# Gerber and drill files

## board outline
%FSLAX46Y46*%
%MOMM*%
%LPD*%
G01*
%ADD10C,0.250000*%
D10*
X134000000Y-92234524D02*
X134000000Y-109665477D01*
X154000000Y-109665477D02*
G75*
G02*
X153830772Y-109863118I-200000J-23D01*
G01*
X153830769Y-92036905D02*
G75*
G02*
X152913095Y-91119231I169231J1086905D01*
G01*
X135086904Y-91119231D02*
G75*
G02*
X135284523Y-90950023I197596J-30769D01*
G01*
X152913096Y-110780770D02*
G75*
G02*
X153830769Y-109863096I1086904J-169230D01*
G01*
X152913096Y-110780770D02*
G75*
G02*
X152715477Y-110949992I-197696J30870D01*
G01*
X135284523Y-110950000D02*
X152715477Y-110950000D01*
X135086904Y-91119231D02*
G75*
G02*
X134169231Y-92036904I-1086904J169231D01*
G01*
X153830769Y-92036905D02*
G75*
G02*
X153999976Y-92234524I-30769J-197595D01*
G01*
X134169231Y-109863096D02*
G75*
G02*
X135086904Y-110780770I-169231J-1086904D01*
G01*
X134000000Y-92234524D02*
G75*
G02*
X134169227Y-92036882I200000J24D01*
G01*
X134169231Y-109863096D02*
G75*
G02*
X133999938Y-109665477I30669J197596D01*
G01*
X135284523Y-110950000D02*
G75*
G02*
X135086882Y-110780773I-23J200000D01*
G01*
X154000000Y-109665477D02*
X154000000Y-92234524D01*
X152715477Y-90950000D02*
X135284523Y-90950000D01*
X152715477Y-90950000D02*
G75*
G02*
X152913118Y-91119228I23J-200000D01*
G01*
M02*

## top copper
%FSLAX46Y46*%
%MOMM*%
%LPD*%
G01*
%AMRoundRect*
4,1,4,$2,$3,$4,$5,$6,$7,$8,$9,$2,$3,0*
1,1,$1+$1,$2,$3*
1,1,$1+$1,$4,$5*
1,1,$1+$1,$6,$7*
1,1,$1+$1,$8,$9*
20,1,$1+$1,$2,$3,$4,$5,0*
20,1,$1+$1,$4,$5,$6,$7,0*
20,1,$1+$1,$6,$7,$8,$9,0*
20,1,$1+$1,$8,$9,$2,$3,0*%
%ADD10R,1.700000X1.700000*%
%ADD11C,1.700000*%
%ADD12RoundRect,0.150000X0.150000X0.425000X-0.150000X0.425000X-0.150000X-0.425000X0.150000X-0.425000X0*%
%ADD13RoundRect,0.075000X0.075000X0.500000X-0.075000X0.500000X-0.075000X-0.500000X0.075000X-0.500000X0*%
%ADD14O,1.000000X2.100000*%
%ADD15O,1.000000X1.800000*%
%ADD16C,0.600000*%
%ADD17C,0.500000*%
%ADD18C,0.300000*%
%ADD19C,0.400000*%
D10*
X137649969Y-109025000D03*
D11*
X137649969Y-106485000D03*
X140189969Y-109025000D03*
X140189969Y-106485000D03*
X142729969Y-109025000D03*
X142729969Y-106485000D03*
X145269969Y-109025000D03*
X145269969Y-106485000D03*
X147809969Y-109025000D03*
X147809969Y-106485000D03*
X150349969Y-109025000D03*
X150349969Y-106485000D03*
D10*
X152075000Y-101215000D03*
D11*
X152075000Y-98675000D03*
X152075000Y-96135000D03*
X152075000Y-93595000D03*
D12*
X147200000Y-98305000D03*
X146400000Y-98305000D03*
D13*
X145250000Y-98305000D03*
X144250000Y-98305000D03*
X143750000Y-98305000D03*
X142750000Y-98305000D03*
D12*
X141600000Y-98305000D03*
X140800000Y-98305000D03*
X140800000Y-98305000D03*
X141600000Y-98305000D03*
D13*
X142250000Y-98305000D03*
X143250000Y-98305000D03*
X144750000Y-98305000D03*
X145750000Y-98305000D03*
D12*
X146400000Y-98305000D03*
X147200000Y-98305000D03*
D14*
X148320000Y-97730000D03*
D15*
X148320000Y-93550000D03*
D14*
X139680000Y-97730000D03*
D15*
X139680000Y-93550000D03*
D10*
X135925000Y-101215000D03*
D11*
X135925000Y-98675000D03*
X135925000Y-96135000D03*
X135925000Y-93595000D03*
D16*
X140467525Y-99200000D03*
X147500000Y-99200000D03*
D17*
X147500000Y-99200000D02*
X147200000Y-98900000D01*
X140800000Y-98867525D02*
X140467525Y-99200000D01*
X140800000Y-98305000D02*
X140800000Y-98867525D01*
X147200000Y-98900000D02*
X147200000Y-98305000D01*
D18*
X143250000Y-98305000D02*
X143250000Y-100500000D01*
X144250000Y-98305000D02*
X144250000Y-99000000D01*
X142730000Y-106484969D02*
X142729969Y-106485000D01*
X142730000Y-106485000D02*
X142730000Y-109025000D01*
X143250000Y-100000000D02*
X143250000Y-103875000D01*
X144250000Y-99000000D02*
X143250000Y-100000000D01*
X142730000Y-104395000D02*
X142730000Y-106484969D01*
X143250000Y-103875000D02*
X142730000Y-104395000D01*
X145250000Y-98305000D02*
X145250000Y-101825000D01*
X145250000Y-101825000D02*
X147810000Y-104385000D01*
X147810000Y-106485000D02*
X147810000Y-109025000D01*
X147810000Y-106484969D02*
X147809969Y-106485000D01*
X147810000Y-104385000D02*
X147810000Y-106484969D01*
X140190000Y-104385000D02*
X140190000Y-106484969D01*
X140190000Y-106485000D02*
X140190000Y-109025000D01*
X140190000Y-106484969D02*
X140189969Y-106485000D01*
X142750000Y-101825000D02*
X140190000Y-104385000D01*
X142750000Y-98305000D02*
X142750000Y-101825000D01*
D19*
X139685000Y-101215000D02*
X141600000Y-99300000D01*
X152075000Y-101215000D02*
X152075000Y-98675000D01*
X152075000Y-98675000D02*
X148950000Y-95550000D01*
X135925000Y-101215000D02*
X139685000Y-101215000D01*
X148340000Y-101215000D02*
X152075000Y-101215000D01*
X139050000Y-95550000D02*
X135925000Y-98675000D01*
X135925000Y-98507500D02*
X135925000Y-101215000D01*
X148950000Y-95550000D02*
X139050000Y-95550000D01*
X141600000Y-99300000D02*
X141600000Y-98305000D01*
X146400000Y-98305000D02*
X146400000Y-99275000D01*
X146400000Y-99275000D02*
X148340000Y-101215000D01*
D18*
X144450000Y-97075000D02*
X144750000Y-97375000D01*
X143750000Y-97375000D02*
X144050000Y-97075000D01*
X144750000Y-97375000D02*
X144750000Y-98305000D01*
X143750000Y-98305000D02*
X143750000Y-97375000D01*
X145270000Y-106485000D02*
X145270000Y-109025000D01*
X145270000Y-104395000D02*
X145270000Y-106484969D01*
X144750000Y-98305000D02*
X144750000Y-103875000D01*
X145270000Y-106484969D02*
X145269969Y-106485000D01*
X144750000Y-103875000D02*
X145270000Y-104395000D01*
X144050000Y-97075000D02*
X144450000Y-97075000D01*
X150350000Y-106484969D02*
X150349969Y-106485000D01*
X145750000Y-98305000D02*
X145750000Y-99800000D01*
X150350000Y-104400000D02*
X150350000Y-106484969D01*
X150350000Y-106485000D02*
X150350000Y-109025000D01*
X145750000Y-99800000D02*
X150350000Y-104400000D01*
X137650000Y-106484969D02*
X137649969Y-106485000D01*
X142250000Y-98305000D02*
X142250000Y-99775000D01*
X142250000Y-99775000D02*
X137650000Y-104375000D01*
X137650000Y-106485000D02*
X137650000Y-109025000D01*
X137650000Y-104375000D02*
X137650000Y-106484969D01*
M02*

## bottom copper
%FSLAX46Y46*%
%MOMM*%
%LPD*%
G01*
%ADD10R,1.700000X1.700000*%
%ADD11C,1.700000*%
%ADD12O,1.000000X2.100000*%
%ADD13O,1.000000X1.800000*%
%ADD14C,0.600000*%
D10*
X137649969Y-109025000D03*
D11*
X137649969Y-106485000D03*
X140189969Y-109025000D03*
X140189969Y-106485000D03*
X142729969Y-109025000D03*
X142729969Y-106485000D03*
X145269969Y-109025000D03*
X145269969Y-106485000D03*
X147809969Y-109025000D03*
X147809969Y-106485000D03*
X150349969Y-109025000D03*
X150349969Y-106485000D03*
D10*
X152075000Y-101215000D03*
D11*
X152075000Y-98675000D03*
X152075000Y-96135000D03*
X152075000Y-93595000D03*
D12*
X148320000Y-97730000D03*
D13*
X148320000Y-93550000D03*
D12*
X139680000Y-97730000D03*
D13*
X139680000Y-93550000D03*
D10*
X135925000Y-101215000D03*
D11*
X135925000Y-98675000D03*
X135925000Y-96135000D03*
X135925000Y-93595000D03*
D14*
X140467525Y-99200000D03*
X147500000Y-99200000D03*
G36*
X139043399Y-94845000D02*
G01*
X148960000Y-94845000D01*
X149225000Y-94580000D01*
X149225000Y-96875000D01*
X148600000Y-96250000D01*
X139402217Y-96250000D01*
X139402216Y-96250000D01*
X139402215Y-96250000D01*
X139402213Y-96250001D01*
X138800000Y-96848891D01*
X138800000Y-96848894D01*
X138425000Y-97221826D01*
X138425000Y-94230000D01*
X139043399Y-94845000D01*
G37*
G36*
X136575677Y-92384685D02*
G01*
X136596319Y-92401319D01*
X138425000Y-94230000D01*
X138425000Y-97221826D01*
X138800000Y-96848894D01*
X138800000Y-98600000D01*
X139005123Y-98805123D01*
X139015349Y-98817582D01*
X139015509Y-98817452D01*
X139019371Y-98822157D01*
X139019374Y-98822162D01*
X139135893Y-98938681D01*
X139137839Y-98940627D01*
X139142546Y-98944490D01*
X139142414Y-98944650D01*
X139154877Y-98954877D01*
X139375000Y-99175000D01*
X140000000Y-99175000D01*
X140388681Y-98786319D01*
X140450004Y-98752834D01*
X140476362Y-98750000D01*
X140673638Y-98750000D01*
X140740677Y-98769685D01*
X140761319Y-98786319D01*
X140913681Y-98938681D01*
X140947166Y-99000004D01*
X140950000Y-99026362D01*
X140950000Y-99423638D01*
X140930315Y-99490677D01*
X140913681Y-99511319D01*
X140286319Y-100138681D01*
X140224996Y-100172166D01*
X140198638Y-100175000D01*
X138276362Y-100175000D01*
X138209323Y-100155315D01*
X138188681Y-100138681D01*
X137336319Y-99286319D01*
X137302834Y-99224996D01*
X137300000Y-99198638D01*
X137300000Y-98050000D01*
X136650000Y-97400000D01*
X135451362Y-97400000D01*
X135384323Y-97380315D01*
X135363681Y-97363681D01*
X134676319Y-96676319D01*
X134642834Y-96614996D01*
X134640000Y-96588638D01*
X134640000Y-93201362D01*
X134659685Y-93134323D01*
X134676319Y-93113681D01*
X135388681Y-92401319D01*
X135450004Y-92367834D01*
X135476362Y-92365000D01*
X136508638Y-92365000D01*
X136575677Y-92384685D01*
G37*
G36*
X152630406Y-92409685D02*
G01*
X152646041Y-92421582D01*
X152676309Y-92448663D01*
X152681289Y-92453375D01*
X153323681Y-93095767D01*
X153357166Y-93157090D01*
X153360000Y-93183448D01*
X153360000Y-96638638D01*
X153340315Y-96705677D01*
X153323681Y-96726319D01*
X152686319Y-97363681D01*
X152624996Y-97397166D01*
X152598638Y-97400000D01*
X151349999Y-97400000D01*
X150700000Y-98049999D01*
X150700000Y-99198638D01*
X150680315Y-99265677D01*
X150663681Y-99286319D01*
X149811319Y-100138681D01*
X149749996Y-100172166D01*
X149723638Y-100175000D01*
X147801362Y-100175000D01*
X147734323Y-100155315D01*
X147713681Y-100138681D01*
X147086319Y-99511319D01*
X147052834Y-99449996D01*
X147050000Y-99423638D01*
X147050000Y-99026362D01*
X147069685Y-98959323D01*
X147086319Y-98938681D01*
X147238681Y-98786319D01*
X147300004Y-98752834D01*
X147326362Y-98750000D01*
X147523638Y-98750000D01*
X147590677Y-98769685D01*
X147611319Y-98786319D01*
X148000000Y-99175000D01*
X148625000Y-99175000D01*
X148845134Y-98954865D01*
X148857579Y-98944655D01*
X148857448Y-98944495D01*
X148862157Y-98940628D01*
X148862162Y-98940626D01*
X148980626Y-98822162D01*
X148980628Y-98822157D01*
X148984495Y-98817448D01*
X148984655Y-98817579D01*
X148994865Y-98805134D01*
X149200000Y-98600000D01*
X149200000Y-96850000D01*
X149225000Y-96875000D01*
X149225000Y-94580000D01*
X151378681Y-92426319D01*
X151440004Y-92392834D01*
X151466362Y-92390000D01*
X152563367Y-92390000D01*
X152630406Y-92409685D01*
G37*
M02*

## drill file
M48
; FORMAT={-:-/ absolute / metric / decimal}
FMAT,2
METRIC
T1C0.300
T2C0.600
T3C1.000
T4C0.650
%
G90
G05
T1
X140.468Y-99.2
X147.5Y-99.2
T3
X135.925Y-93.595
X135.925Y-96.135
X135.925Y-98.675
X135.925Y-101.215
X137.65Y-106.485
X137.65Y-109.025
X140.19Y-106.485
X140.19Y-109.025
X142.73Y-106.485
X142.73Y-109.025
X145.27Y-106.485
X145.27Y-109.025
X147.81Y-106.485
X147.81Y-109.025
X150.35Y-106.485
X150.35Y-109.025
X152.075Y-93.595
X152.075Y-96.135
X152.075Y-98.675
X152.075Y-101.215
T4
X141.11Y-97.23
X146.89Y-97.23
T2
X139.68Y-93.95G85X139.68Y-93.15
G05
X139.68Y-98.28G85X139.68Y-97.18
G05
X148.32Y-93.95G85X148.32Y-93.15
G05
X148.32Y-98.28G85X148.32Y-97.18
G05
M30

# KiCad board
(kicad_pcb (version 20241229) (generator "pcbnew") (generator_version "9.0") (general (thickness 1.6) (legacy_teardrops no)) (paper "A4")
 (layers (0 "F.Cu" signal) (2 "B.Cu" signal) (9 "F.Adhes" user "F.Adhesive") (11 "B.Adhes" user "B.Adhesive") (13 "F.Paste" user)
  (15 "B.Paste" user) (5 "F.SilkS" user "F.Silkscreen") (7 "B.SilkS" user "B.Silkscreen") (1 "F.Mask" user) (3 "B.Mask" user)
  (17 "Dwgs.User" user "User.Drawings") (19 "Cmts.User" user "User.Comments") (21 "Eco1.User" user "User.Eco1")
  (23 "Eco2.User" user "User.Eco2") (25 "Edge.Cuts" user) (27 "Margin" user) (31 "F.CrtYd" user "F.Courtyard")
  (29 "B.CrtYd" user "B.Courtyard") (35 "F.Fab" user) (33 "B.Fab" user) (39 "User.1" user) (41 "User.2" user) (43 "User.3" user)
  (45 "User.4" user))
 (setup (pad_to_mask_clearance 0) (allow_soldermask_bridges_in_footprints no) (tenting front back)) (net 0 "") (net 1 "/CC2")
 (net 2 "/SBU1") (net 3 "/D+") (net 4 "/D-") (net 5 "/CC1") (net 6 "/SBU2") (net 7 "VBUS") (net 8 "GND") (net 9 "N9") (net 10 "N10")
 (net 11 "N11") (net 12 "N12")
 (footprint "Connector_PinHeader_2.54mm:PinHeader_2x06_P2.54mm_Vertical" (layer "F.Cu") (at 137.649969 109.025 90)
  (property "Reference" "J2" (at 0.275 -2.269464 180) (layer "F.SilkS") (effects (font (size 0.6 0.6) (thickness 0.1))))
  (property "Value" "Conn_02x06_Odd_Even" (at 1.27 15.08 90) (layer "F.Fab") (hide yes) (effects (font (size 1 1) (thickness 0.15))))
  (pad "1" thru_hole rect (at 0 0 90) (size 1.7 1.7) (drill 1) (layers "*.Cu" "*.Mask") (remove_unused_layers no) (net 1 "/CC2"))
  (pad "2" thru_hole circle (at 2.54 0 90) (size 1.7 1.7) (drill 1) (layers "*.Cu" "*.Mask") (remove_unused_layers no) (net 1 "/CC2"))
  (pad "3" thru_hole circle (at 0 2.54 90) (size 1.7 1.7) (drill 1) (layers "*.Cu" "*.Mask") (remove_unused_layers no) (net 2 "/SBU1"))
  (pad "4" thru_hole circle (at 2.54 2.54 90) (size 1.7 1.7) (drill 1) (layers "*.Cu" "*.Mask") (remove_unused_layers no) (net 2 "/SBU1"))
  (pad "5" thru_hole circle (at 0 5.08 90) (size 1.7 1.7) (drill 1) (layers "*.Cu" "*.Mask") (remove_unused_layers no) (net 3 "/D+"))
  (pad "6" thru_hole circle (at 2.54 5.08 90) (size 1.7 1.7) (drill 1) (layers "*.Cu" "*.Mask") (remove_unused_layers no) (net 3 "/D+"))
  (pad "7" thru_hole circle (at 0 7.62 90) (size 1.7 1.7) (drill 1) (layers "*.Cu" "*.Mask") (remove_unused_layers no) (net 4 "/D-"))
  (pad "8" thru_hole circle (at 2.54 7.62 90) (size 1.7 1.7) (drill 1) (layers "*.Cu" "*.Mask") (remove_unused_layers no) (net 4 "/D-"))
  (pad "9" thru_hole circle (at 0 10.16 90) (size 1.7 1.7) (drill 1) (layers "*.Cu" "*.Mask") (remove_unused_layers no) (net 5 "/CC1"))
  (pad "10" thru_hole circle (at 2.54 10.16 90) (size 1.7 1.7) (drill 1) (layers "*.Cu" "*.Mask") (remove_unused_layers no) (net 5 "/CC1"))
  (pad "11" thru_hole circle (at 0 12.7 90) (size 1.7 1.7) (drill 1) (layers "*.Cu" "*.Mask") (remove_unused_layers no) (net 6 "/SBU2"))
  (pad "12" thru_hole circle (at 2.54 12.7 90) (size 1.7 1.7) (drill 1) (layers "*.Cu" "*.Mask") (remove_unused_layers no) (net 6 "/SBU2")))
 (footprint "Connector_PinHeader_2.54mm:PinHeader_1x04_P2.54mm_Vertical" (layer "F.Cu") (at 152.075 101.215 180)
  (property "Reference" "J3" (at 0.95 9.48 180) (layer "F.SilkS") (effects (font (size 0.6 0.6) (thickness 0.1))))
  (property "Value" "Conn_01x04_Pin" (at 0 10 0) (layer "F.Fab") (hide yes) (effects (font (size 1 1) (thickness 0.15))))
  (pad "1" thru_hole rect (at 0 0 180) (size 1.7 1.7) (drill 1) (layers "*.Cu" "*.Mask") (remove_unused_layers no) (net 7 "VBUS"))
  (pad "2" thru_hole circle (at 0 2.54 180) (size 1.7 1.7) (drill 1) (layers "*.Cu" "*.Mask") (remove_unused_layers no) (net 7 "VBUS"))
  (pad "3" thru_hole circle (at 0 5.08 180) (size 1.7 1.7) (drill 1) (layers "*.Cu" "*.Mask") (remove_unused_layers no) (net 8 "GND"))
  (pad "4" thru_hole circle (at 0 7.62 180) (size 1.7 1.7) (drill 1) (layers "*.Cu" "*.Mask") (remove_unused_layers no) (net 8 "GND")))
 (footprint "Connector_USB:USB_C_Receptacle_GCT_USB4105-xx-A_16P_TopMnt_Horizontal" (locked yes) (layer "F.Cu") (at 144 94.625 180)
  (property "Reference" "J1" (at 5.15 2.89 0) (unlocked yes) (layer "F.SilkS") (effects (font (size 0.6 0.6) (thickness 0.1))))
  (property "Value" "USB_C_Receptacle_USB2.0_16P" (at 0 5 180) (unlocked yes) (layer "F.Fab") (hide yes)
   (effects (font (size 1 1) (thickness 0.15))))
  (pad "" np_thru_hole circle (at -2.89 -2.605 180) (size 0.65 0.65) (drill 0.65) (layers "*.Cu" "*.Mask"))
  (pad "" np_thru_hole circle (at 2.89 -2.605 180) (size 0.65 0.65) (drill 0.65) (layers "*.Cu" "*.Mask"))
  (pad "A1" smd roundrect (at -3.2 -3.68 180) (size 0.6 1.15) (layers "F.Cu" "F.Mask" "F.Paste") (roundrect_rratio 0.25) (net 8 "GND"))
  (pad "A4" smd roundrect (at -2.4 -3.68 180) (size 0.6 1.15) (layers "F.Cu" "F.Mask" "F.Paste") (roundrect_rratio 0.25) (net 7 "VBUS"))
  (pad "A5" smd roundrect (at -1.25 -3.68 180) (size 0.3 1.15) (layers "F.Cu" "F.Mask" "F.Paste") (roundrect_rratio 0.25) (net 5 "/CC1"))
  (pad "A6" smd roundrect (at -0.25 -3.68 180) (size 0.3 1.15) (layers "F.Cu" "F.Mask" "F.Paste") (roundrect_rratio 0.25) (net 3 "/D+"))
  (pad "A7" smd roundrect (at 0.25 -3.68 180) (size 0.3 1.15) (layers "F.Cu" "F.Mask" "F.Paste") (roundrect_rratio 0.25) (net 4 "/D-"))
  (pad "A8" smd roundrect (at 1.25 -3.68 180) (size 0.3 1.15) (layers "F.Cu" "F.Mask" "F.Paste") (roundrect_rratio 0.25) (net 2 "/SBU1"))
  (pad "A9" smd roundrect (at 2.4 -3.68 180) (size 0.6 1.15) (layers "F.Cu" "F.Mask" "F.Paste") (roundrect_rratio 0.25) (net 7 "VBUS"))
  (pad "A12" smd roundrect (at 3.2 -3.68 180) (size 0.6 1.15) (layers "F.Cu" "F.Mask" "F.Paste") (roundrect_rratio 0.25) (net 8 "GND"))
  (pad "B1" smd roundrect (at 3.2 -3.68 180) (size 0.6 1.15) (layers "F.Cu" "F.Mask" "F.Paste") (roundrect_rratio 0.25) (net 8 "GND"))
  (pad "B4" smd roundrect (at 2.4 -3.68 180) (size 0.6 1.15) (layers "F.Cu" "F.Mask" "F.Paste") (roundrect_rratio 0.25) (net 7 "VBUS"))
  (pad "B5" smd roundrect (at 1.75 -3.68 180) (size 0.3 1.15) (layers "F.Cu" "F.Mask" "F.Paste") (roundrect_rratio 0.25) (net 1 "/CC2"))
  (pad "B6" smd roundrect (at 0.75 -3.68 180) (size 0.3 1.15) (layers "F.Cu" "F.Mask" "F.Paste") (roundrect_rratio 0.25) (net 3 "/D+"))
  (pad "B7" smd roundrect (at -0.75 -3.68 180) (size 0.3 1.15) (layers "F.Cu" "F.Mask" "F.Paste") (roundrect_rratio 0.25) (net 4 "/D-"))
  (pad "B8" smd roundrect (at -1.75 -3.68 180) (size 0.3 1.15) (layers "F.Cu" "F.Mask" "F.Paste") (roundrect_rratio 0.25) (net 6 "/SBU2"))
  (pad "B9" smd roundrect (at -2.4 -3.68 180) (size 0.6 1.15) (layers "F.Cu" "F.Mask" "F.Paste") (roundrect_rratio 0.25) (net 7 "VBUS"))
  (pad "B12" smd roundrect (at -3.2 -3.68 180) (size 0.6 1.15) (layers "F.Cu" "F.Mask" "F.Paste") (roundrect_rratio 0.25) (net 8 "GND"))
  (pad "S1" thru_hole oval (at -4.32 -3.105 180) (size 1 2.1) (drill oval 0.6 1.7) (layers "*.Cu" "*.Mask" "F.Paste")
   (remove_unused_layers no) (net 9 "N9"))
  (pad "S1" thru_hole oval (at -4.32 1.075 180) (size 1 1.8) (drill oval 0.6 1.4) (layers "*.Cu" "*.Mask" "F.Paste")
   (remove_unused_layers no) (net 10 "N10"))
  (pad "S1" thru_hole oval (at 4.32 -3.105 180) (size 1 2.1) (drill oval 0.6 1.7) (layers "*.Cu" "*.Mask" "F.Paste")
   (remove_unused_layers no) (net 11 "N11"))
  (pad "S1" thru_hole oval (at 4.32 1.075 180) (size 1 1.8) (drill oval 0.6 1.4) (layers "*.Cu" "*.Mask" "F.Paste")
   (remove_unused_layers no) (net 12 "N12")))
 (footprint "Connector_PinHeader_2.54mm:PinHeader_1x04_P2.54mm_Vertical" (layer "F.Cu") (at 135.925 101.215 180)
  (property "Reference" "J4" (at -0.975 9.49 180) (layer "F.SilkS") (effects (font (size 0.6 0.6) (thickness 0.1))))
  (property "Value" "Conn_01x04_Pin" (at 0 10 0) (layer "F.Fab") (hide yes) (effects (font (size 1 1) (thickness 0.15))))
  (pad "1" thru_hole rect (at 0 0 180) (size 1.7 1.7) (drill 1) (layers "*.Cu" "*.Mask") (remove_unused_layers no) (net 7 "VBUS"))
  (pad "2" thru_hole circle (at 0 2.54 180) (size 1.7 1.7) (drill 1) (layers "*.Cu" "*.Mask") (remove_unused_layers no) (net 7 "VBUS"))
  (pad "3" thru_hole circle (at 0 5.08 180) (size 1.7 1.7) (drill 1) (layers "*.Cu" "*.Mask") (remove_unused_layers no) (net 8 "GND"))
  (pad "4" thru_hole circle (at 0 7.62 180) (size 1.7 1.7) (drill 1) (layers "*.Cu" "*.Mask") (remove_unused_layers no) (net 8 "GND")))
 (gr_line (start 134 92.234524) (end 134 109.665477) (stroke (width 0.25) (type solid)) (locked yes) (layer "Edge.Cuts"))
 (gr_arc (start 154 109.665477) (mid 153.951919 109.795579) (end 153.830769 109.863096) (stroke (width 0.25) (type solid)) (locked yes)
  (layer "Edge.Cuts"))
 (gr_arc (start 153.830769 92.036905) (mid 153.222182 91.727818) (end 152.913096 91.119231) (stroke (width 0.25) (type solid)) (locked yes)
  (layer "Edge.Cuts"))
 (gr_arc (start 135.086904 91.119231) (mid 135.154436 90.998098) (end 135.284523 90.95) (stroke (width 0.25) (type solid)) (locked yes)
  (layer "Edge.Cuts"))
 (gr_arc (start 152.913096 110.78077) (mid 153.222182 110.172183) (end 153.830769 109.863096) (stroke (width 0.25) (type solid))
  (locked yes) (layer "Edge.Cuts"))
 (gr_arc (start 152.913096 110.78077) (mid 152.845544 110.901884) (end 152.715477 110.95) (stroke (width 0.25) (type solid)) (locked yes)
  (layer "Edge.Cuts"))
 (gr_line (start 135.284523 110.95) (end 152.715477 110.95) (stroke (width 0.25) (type solid)) (locked yes) (layer "Edge.Cuts"))
 (gr_arc (start 135.086904 91.119231) (mid 134.777817 91.727817) (end 134.169231 92.036905) (stroke (width 0.25) (type solid)) (locked yes)
  (layer "Edge.Cuts"))
 (gr_arc (start 153.830769 92.036905) (mid 153.951902 92.104437) (end 154 92.234524) (stroke (width 0.25) (type solid)) (locked yes)
  (layer "Edge.Cuts"))
 (gr_arc (start 134.169231 109.863096) (mid 134.777818 110.172183) (end 135.086904 110.78077) (stroke (width 0.25) (type solid))
  (locked yes) (layer "Edge.Cuts"))
 (gr_arc (start 134 92.234524) (mid 134.048088 92.104449) (end 134.169231 92.036905) (stroke (width 0.25) (type solid)) (locked yes)
  (layer "Edge.Cuts"))
 (gr_arc (start 134.169231 109.863096) (mid 134.04806 109.795572) (end 134 109.665477) (stroke (width 0.25) (type solid)) (locked yes)
  (layer "Edge.Cuts"))
 (gr_arc (start 135.284523 110.95) (mid 135.154422 110.90192) (end 135.086904 110.78077) (stroke (width 0.25) (type solid)) (locked yes)
  (layer "Edge.Cuts"))
 (gr_line (start 154 109.665477) (end 154 92.234524) (stroke (width 0.25) (type solid)) (locked yes) (layer "Edge.Cuts"))
 (gr_line (start 152.715477 90.95) (end 135.284523 90.95) (stroke (width 0.25) (type solid)) (locked yes) (layer "Edge.Cuts"))
 (gr_arc (start 152.715477 90.95) (mid 152.845551 90.998089) (end 152.913096 91.119231) (stroke (width 0.25) (type solid)) (locked yes)
  (layer "Edge.Cuts"))
 (segment (start 147.5 99.2) (end 147.2 98.9) (width 0.5) (layer "F.Cu") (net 8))
 (segment (start 140.8 98.867525) (end 140.467525 99.2) (width 0.5) (layer "F.Cu") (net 8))
 (segment (start 140.8 98.305) (end 140.8 98.867525) (width 0.5) (layer "F.Cu") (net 8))
 (segment (start 147.2 98.9) (end 147.2 98.305) (width 0.5) (layer "F.Cu") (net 8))
 (via (at 140.467525 99.2) (size 0.6) (drill 0.3) (layers "F.Cu" "B.Cu") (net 8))
 (via (at 147.5 99.2) (size 0.6) (drill 0.3) (layers "F.Cu" "B.Cu") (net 8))
 (segment (start 143.25 98.305) (end 143.25 100.5) (width 0.3) (layer "F.Cu") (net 3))
 (segment (start 144.25 98.305) (end 144.25 99) (width 0.3) (layer "F.Cu") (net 3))
 (segment (start 142.73 106.484969) (end 142.729969 106.485) (width 0.3) (layer "F.Cu") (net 3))
 (segment (start 142.73 106.485) (end 142.73 109.025) (width 0.3) (layer "F.Cu") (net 3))
 (segment (start 143.25 100) (end 143.25 103.875) (width 0.3) (layer "F.Cu") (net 3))
 (segment (start 144.25 99) (end 143.25 100) (width 0.3) (layer "F.Cu") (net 3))
 (segment (start 142.73 104.395) (end 142.73 106.484969) (width 0.3) (layer "F.Cu") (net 3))
 (segment (start 143.25 103.875) (end 142.73 104.395) (width 0.3) (layer "F.Cu") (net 3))
 (segment (start 145.25 98.305) (end 145.25 101.825) (width 0.3) (layer "F.Cu") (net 5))
 (segment (start 145.25 101.825) (end 147.81 104.385) (width 0.3) (layer "F.Cu") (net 5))
 (segment (start 147.81 106.485) (end 147.81 109.025) (width 0.3) (layer "F.Cu") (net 5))
 (segment (start 147.81 106.484969) (end 147.809969 106.485) (width 0.3) (layer "F.Cu") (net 5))
 (segment (start 147.81 104.385) (end 147.81 106.484969) (width 0.3) (layer "F.Cu") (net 5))
 (segment (start 140.19 104.385) (end 140.19 106.484969) (width 0.3) (layer "F.Cu") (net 2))
 (segment (start 140.19 106.485) (end 140.19 109.025) (width 0.3) (layer "F.Cu") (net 2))
 (segment (start 140.19 106.484969) (end 140.189969 106.485) (width 0.3) (layer "F.Cu") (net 2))
 (segment (start 142.75 101.825) (end 140.19 104.385) (width 0.3) (layer "F.Cu") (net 2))
 (segment (start 142.75 98.305) (end 142.75 101.825) (width 0.3) (layer "F.Cu") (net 2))
 (segment (start 139.685 101.215) (end 141.6 99.3) (width 0.4) (layer "F.Cu") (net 7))
 (segment (start 152.075 101.215) (end 152.075 98.675) (width 0.4) (layer "F.Cu") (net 7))
 (segment (start 152.075 98.675) (end 148.95 95.55) (width 0.4) (layer "F.Cu") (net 7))
 (segment (start 135.925 101.215) (end 139.685 101.215) (width 0.4) (layer "F.Cu") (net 7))
 (segment (start 148.34 101.215) (end 152.075 101.215) (width 0.4) (layer "F.Cu") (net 7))
 (segment (start 139.05 95.55) (end 135.925 98.675) (width 0.4) (layer "F.Cu") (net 7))
 (segment (start 135.925 98.5075) (end 135.925 101.215) (width 0.4) (layer "F.Cu") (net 7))
 (segment (start 148.95 95.55) (end 139.05 95.55) (width 0.4) (layer "F.Cu") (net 7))
 (segment (start 141.6 99.3) (end 141.6 98.305) (width 0.4) (layer "F.Cu") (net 7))
 (segment (start 146.4 98.305) (end 146.4 99.275) (width 0.4) (layer "F.Cu") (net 7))
 (segment (start 146.4 99.275) (end 148.34 101.215) (width 0.4) (layer "F.Cu") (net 7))
 (segment (start 144.45 97.075) (end 144.75 97.375) (width 0.3) (layer "F.Cu") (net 4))
 (segment (start 143.75 97.375) (end 144.05 97.075) (width 0.3) (layer "F.Cu") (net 4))
 (segment (start 144.75 97.375) (end 144.75 98.305) (width 0.3) (layer "F.Cu") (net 4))
 (segment (start 143.75 98.305) (end 143.75 97.375) (width 0.3) (layer "F.Cu") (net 4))
 (segment (start 145.27 106.485) (end 145.27 109.025) (width 0.3) (layer "F.Cu") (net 4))
 (segment (start 145.27 104.395) (end 145.27 106.484969) (width 0.3) (layer "F.Cu") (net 4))
 (segment (start 144.75 98.305) (end 144.75 103.875) (width 0.3) (layer "F.Cu") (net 4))
 (segment (start 145.27 106.484969) (end 145.269969 106.485) (width 0.3) (layer "F.Cu") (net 4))
 (segment (start 144.75 103.875) (end 145.27 104.395) (width 0.3) (layer "F.Cu") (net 4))
 (segment (start 144.05 97.075) (end 144.45 97.075) (width 0.3) (layer "F.Cu") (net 4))
 (segment (start 150.35 106.484969) (end 150.349969 106.485) (width 0.3) (layer "F.Cu") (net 6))
 (segment (start 145.75 98.305) (end 145.75 99.8) (width 0.3) (layer "F.Cu") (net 6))
 (segment (start 150.35 104.4) (end 150.35 106.484969) (width 0.3) (layer "F.Cu") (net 6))
 (segment (start 150.35 106.485) (end 150.35 109.025) (width 0.3) (layer "F.Cu") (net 6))
 (segment (start 145.75 99.8) (end 150.35 104.4) (width 0.3) (layer "F.Cu") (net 6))
 (segment (start 137.65 106.484969) (end 137.649969 106.485) (width 0.3) (layer "F.Cu") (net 1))
 (segment (start 142.25 98.305) (end 142.25 99.775) (width 0.3) (layer "F.Cu") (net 1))
 (segment (start 142.25 99.775) (end 137.65 104.375) (width 0.3) (layer "F.Cu") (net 1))
 (segment (start 137.65 106.485) (end 137.65 109.025) (width 0.3) (layer "F.Cu") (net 1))
 (segment (start 137.65 104.375) (end 137.65 106.484969) (width 0.3) (layer "F.Cu") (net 1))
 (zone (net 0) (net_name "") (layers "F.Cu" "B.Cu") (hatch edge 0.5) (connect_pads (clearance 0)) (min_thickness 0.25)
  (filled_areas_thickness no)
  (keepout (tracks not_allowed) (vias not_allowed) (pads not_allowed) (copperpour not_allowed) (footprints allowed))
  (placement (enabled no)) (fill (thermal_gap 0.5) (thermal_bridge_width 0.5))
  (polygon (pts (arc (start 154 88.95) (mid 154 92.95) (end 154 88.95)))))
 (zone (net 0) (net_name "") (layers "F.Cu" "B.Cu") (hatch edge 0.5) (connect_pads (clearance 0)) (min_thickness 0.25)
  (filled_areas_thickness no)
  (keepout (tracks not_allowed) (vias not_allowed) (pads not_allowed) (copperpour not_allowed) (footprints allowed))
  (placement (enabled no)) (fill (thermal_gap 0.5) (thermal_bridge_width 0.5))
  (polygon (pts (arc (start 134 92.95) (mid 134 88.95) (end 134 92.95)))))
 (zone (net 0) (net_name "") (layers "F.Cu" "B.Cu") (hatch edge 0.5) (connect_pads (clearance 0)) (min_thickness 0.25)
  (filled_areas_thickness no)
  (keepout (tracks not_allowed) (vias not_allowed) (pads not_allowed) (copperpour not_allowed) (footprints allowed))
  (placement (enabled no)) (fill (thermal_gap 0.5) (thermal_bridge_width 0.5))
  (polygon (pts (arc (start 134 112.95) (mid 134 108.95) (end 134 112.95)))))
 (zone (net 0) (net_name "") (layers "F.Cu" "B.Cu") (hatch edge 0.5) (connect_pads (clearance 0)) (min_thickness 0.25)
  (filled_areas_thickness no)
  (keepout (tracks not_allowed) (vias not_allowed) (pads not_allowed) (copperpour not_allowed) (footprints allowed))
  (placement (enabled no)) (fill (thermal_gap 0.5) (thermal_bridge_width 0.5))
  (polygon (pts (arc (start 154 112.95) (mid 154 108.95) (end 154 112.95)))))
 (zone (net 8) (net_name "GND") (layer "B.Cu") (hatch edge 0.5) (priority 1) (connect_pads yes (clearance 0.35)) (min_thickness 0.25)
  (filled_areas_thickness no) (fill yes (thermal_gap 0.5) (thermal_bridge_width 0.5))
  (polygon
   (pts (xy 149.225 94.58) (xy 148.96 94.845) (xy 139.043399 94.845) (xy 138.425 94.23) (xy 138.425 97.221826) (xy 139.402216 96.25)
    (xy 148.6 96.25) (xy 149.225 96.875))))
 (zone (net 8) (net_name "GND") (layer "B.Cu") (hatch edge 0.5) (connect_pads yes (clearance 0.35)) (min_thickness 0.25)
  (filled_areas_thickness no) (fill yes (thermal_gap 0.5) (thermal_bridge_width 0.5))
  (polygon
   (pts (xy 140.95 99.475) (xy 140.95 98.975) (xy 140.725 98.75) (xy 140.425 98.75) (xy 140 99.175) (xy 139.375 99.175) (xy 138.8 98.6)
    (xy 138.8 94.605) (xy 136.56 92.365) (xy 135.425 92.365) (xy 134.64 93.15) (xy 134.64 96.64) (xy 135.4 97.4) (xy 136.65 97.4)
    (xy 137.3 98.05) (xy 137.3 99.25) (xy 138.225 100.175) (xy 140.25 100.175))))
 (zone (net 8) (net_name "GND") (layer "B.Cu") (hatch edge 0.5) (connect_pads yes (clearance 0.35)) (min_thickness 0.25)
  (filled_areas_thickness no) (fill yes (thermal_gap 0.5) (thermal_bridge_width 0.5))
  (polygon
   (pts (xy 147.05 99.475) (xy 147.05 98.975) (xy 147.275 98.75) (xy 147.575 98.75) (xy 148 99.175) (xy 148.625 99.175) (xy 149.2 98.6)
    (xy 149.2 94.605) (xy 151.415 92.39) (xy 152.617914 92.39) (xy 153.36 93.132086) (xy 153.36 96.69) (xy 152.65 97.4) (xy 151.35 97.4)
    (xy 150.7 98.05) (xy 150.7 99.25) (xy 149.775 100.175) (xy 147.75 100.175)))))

